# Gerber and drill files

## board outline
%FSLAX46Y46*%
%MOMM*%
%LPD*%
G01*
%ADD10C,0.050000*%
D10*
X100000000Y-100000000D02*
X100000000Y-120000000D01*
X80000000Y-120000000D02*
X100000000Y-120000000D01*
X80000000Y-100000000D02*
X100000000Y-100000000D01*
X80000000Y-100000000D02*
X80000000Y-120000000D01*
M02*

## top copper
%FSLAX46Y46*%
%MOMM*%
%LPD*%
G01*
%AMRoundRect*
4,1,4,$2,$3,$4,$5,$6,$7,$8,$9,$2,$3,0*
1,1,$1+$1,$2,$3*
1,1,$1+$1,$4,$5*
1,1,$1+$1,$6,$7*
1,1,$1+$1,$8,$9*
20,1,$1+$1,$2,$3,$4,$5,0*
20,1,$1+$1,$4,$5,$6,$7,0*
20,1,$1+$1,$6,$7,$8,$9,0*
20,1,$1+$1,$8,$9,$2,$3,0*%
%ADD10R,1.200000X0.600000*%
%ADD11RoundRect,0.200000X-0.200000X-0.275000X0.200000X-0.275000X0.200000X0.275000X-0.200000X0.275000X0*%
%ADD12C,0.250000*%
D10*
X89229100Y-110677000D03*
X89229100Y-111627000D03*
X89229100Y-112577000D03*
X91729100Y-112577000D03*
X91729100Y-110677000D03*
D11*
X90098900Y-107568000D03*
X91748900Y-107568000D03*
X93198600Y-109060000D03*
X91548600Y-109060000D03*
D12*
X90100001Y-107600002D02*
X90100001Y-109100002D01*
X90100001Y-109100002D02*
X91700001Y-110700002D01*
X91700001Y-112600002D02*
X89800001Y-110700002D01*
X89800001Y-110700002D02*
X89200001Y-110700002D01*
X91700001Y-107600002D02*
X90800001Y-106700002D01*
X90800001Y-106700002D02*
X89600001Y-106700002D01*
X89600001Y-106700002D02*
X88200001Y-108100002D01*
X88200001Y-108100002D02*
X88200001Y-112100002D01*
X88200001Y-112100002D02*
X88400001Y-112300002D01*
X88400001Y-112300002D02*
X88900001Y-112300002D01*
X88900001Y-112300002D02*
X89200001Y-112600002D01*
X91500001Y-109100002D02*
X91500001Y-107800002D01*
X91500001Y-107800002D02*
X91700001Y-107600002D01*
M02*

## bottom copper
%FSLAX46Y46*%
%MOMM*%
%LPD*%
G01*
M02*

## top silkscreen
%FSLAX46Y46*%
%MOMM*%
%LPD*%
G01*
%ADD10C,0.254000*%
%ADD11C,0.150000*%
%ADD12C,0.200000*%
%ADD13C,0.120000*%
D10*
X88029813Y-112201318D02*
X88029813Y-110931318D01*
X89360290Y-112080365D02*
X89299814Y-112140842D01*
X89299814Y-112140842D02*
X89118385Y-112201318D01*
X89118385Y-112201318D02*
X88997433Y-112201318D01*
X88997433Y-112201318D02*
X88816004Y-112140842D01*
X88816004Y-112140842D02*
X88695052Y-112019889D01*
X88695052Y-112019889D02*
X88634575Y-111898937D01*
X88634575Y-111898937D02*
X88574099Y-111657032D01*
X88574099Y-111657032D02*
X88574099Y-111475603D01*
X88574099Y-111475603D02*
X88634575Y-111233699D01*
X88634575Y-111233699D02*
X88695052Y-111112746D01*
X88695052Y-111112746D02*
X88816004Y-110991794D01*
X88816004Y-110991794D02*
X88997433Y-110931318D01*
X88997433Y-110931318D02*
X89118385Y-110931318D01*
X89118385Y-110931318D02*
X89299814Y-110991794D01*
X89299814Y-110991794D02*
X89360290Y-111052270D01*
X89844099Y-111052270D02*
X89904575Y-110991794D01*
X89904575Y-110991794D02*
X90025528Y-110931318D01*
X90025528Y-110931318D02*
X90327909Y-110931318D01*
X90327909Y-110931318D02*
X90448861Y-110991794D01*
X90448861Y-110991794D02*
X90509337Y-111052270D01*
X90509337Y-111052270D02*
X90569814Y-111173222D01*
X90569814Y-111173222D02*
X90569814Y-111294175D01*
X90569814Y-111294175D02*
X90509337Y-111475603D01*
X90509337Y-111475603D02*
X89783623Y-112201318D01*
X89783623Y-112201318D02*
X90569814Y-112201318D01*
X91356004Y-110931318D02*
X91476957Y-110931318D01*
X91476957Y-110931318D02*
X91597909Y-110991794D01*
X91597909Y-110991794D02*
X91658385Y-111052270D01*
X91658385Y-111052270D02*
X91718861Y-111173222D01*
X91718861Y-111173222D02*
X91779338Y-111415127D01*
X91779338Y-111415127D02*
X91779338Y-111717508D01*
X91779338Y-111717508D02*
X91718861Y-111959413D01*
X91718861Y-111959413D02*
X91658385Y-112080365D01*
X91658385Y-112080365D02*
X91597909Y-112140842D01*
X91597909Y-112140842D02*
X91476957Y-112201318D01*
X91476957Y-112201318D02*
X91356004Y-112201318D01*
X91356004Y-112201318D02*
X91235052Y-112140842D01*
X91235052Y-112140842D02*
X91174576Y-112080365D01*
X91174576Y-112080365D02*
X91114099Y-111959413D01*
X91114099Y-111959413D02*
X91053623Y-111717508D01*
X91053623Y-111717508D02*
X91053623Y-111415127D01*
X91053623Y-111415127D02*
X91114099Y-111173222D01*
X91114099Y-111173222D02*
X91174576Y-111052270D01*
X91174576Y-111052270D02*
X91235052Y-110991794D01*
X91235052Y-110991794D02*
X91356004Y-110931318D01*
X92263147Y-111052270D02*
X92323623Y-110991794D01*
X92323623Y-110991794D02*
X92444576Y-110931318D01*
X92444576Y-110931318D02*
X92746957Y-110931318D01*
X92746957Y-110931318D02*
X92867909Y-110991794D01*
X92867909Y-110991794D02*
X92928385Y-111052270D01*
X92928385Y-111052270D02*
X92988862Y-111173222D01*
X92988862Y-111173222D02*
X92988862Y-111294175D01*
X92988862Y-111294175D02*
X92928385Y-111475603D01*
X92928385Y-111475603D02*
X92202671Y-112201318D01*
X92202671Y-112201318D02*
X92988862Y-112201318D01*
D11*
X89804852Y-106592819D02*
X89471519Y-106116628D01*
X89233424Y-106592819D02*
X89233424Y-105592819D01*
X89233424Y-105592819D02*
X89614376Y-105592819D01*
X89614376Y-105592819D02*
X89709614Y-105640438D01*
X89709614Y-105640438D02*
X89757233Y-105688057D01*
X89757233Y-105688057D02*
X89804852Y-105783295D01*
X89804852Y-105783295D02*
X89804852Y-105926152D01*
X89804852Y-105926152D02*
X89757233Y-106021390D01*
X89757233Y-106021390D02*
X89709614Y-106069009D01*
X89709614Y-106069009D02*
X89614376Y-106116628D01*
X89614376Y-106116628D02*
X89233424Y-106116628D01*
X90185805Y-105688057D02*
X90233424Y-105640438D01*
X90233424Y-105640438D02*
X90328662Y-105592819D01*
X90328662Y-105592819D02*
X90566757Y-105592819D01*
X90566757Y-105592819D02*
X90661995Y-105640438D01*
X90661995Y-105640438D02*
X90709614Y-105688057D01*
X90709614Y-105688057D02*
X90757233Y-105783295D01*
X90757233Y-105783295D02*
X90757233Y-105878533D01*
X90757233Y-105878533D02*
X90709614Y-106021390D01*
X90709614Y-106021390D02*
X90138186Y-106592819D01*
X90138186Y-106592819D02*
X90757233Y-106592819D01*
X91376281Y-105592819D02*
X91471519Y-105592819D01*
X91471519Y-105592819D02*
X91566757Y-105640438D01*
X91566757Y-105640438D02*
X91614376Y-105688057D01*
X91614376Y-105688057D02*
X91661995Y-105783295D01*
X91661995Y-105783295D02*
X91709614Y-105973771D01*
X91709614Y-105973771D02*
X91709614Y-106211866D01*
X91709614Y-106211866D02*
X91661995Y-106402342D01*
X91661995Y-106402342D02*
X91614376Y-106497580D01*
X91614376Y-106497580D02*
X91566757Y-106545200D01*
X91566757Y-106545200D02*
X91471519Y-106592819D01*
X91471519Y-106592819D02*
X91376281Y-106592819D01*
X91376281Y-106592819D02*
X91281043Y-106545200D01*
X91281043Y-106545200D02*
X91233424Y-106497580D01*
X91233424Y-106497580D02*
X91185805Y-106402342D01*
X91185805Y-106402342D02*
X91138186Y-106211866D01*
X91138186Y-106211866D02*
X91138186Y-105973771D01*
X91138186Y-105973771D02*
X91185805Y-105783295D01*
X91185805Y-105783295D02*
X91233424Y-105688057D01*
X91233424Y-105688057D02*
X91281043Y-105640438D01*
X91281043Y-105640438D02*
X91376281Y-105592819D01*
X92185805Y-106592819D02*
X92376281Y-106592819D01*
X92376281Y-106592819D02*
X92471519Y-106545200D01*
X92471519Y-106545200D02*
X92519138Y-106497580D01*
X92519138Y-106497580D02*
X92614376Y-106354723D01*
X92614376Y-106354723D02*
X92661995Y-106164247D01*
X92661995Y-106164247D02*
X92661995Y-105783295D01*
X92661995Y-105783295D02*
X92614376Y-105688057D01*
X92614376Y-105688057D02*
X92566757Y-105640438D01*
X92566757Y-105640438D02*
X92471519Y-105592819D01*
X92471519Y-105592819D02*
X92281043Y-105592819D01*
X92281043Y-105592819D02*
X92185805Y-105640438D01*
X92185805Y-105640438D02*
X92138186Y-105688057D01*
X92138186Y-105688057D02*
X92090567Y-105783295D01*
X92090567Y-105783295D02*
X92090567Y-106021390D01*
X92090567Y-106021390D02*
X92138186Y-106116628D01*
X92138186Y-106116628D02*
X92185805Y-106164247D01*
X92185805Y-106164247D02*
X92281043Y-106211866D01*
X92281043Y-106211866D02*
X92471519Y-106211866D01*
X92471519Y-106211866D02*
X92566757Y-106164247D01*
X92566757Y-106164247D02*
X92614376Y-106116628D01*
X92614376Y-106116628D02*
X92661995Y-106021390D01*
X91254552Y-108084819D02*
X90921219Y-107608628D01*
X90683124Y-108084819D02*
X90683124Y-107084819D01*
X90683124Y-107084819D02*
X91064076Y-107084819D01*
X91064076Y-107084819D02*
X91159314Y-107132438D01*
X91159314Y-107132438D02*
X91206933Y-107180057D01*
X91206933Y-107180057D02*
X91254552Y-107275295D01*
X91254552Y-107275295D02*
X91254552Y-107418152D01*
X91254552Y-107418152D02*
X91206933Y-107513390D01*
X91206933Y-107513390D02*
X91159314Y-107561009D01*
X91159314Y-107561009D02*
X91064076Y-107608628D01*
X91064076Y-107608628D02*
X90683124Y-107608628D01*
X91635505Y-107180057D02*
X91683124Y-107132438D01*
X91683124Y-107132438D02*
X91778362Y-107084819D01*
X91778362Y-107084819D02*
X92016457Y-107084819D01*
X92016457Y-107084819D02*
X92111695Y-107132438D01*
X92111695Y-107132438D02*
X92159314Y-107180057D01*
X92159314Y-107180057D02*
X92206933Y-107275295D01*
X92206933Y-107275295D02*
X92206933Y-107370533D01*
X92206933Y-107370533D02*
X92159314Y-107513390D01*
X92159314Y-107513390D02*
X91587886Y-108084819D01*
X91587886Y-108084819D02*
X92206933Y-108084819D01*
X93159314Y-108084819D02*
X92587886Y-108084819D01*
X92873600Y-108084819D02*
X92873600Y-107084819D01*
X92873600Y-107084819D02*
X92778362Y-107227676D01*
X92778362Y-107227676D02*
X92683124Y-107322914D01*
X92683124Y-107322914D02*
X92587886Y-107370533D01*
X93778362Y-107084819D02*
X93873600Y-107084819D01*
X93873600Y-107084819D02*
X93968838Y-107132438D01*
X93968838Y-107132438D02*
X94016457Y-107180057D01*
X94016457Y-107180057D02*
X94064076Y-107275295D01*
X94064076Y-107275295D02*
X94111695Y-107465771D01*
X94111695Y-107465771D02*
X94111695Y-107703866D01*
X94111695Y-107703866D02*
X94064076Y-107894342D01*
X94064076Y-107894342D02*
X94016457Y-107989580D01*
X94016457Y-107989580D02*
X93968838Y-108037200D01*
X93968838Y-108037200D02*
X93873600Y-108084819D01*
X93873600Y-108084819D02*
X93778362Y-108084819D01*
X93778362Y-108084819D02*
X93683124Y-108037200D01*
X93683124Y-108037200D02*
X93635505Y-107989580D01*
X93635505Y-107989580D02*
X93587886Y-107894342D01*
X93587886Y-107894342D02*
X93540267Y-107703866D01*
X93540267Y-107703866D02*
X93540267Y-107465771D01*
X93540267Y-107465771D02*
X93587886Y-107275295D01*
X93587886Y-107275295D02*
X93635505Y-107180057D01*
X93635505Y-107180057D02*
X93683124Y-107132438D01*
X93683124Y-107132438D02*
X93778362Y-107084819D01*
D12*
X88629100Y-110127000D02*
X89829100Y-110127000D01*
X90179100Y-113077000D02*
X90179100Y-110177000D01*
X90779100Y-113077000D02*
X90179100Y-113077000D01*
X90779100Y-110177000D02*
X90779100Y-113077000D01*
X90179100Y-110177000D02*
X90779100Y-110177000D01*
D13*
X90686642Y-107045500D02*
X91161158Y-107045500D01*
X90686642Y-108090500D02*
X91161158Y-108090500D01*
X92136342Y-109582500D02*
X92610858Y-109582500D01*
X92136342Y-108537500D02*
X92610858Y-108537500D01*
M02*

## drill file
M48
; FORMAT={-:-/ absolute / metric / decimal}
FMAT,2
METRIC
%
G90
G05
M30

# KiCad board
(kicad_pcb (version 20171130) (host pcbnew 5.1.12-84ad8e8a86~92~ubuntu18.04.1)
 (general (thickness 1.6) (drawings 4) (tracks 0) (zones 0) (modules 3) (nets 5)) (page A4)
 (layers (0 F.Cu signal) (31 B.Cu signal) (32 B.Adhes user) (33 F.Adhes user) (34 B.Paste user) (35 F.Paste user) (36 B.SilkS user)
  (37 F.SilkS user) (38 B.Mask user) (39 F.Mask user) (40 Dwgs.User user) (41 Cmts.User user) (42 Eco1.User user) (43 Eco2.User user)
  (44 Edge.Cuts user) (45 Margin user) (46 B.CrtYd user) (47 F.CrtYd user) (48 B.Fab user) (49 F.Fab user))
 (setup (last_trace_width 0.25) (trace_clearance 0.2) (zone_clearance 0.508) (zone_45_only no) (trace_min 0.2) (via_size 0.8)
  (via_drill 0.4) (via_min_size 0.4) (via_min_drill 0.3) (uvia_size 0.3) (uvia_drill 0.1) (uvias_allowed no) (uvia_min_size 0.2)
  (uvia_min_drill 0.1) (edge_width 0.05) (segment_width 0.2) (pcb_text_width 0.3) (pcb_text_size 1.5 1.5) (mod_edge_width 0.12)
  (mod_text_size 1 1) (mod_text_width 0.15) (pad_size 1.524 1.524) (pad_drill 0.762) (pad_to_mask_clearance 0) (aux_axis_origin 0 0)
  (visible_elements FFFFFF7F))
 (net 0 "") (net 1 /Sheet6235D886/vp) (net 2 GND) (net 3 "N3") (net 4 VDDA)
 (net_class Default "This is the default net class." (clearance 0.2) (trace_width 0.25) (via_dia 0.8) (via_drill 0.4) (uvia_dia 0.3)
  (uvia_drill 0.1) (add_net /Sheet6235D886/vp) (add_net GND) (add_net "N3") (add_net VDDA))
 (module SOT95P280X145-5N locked (layer F.Cu) (at 90.479100 111.627000)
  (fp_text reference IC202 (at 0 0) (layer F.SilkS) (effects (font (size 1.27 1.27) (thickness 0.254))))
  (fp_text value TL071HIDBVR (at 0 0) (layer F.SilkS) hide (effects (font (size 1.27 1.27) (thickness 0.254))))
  (fp_line (start -1.85 -1.5) (end -0.65 -1.5) (layer F.SilkS) (width 0.2))
  (fp_line (start -0.3 1.45) (end -0.3 -1.45) (layer F.SilkS) (width 0.2))
  (fp_line (start 0.3 1.45) (end -0.3 1.45) (layer F.SilkS) (width 0.2))
  (fp_line (start 0.3 -1.45) (end 0.3 1.45) (layer F.SilkS) (width 0.2))
  (fp_line (start -0.3 -1.45) (end 0.3 -1.45) (layer F.SilkS) (width 0.2))
  (pad 1 smd rect (at -1.25 -0.95 90.000000) (size 0.6 1.2) (layers F.Cu F.Mask F.Paste) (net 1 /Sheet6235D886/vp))
  (pad 2 smd rect (at -1.25 0 90.000000) (size 0.6 1.2) (layers F.Cu F.Mask F.Paste) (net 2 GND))
  (pad 3 smd rect (at -1.25 0.95 90.000000) (size 0.6 1.2) (layers F.Cu F.Mask F.Paste) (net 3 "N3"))
  (pad 4 smd rect (at 1.25 0.95 90.000000) (size 0.6 1.2) (layers F.Cu F.Mask F.Paste) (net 1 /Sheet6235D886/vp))
  (pad 5 smd rect (at 1.25 -0.95 90.000000) (size 0.6 1.2) (layers F.Cu F.Mask F.Paste) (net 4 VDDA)))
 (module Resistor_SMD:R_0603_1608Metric (layer F.Cu) (at 90.923900 107.568000)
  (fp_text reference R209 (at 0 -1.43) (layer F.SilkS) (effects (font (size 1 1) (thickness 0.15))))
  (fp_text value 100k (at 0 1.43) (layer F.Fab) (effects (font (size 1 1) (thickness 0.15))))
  (fp_line (start -0.237258 -0.5225) (end 0.237258 -0.5225) (layer F.SilkS) (width 0.12))
  (fp_line (start -0.237258 0.5225) (end 0.237258 0.5225) (layer F.SilkS) (width 0.12))
  (pad 1 smd roundrect (at -0.825 0) (size 0.8 0.95) (layers F.Cu F.Mask F.Paste) (roundrect_rratio 0.25) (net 4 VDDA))
  (pad 2 smd roundrect (at 0.825 0) (size 0.8 0.95) (layers F.Cu F.Mask F.Paste) (roundrect_rratio 0.25) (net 3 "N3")))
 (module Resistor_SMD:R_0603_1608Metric (layer F.Cu) (at 92.373600 109.060000)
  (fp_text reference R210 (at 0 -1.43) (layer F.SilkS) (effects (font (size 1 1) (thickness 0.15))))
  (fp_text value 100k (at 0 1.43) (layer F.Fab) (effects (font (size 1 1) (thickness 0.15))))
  (fp_line (start -0.237258 0.5225) (end 0.237258 0.5225) (layer F.SilkS) (width 0.12))
  (fp_line (start -0.237258 -0.5225) (end 0.237258 -0.5225) (layer F.SilkS) (width 0.12))
  (pad 2 smd roundrect (at 0.825 0) (size 0.8 0.95) (layers F.Cu F.Mask F.Paste) (roundrect_rratio 0.25) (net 2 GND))
  (pad 1 smd roundrect (at -0.825 0) (size 0.8 0.95) (layers F.Cu F.Mask F.Paste) (roundrect_rratio 0.25) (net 3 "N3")))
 (gr_line (start 100 100) (end 100 120) (layer Edge.Cuts) (width 0.05))
 (gr_line (start 80 120) (end 100 120) (layer Edge.Cuts) (width 0.05))
 (gr_line (start 80 100) (end 100 100) (layer Edge.Cuts) (width 0.05))
 (gr_line (start 80 100) (end 80 120) (layer Edge.Cuts) (width 0.05))
 (segment (start 90.100001 107.600002) (end 90.100001 109.100002) (width 0.250000) (layer F.Cu) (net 4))
 (segment (start 90.100001 109.100002) (end 91.700001 110.700002) (width 0.250000) (layer F.Cu) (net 4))
 (segment (start 91.700001 112.600002) (end 89.800001 110.700002) (width 0.250000) (layer F.Cu) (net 1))
 (segment (start 89.800001 110.700002) (end 89.200001 110.700002) (width 0.250000) (layer F.Cu) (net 1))
 (segment (start 91.700001 107.600002) (end 90.800001 106.700002) (width 0.250000) (layer F.Cu) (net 3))
 (segment (start 90.800001 106.700002) (end 89.600001 106.700002) (width 0.250000) (layer F.Cu) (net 3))
 (segment (start 89.600001 106.700002) (end 88.200001 108.100002) (width 0.250000) (layer F.Cu) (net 3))
 (segment (start 88.200001 108.100002) (end 88.200001 112.100002) (width 0.250000) (layer F.Cu) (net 3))
 (segment (start 88.200001 112.100002) (end 88.400001 112.300002) (width 0.250000) (layer F.Cu) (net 3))
 (segment (start 88.400001 112.300002) (end 88.900001 112.300002) (width 0.250000) (layer F.Cu) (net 3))
 (segment (start 88.900001 112.300002) (end 89.200001 112.600002) (width 0.250000) (layer F.Cu) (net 3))
 (segment (start 91.500001 109.100002) (end 91.500001 107.800002) (width 0.250000) (layer F.Cu) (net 3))
 (segment (start 91.500001 107.800002) (end 91.700001 107.600002) (width 0.250000) (layer F.Cu) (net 3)))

